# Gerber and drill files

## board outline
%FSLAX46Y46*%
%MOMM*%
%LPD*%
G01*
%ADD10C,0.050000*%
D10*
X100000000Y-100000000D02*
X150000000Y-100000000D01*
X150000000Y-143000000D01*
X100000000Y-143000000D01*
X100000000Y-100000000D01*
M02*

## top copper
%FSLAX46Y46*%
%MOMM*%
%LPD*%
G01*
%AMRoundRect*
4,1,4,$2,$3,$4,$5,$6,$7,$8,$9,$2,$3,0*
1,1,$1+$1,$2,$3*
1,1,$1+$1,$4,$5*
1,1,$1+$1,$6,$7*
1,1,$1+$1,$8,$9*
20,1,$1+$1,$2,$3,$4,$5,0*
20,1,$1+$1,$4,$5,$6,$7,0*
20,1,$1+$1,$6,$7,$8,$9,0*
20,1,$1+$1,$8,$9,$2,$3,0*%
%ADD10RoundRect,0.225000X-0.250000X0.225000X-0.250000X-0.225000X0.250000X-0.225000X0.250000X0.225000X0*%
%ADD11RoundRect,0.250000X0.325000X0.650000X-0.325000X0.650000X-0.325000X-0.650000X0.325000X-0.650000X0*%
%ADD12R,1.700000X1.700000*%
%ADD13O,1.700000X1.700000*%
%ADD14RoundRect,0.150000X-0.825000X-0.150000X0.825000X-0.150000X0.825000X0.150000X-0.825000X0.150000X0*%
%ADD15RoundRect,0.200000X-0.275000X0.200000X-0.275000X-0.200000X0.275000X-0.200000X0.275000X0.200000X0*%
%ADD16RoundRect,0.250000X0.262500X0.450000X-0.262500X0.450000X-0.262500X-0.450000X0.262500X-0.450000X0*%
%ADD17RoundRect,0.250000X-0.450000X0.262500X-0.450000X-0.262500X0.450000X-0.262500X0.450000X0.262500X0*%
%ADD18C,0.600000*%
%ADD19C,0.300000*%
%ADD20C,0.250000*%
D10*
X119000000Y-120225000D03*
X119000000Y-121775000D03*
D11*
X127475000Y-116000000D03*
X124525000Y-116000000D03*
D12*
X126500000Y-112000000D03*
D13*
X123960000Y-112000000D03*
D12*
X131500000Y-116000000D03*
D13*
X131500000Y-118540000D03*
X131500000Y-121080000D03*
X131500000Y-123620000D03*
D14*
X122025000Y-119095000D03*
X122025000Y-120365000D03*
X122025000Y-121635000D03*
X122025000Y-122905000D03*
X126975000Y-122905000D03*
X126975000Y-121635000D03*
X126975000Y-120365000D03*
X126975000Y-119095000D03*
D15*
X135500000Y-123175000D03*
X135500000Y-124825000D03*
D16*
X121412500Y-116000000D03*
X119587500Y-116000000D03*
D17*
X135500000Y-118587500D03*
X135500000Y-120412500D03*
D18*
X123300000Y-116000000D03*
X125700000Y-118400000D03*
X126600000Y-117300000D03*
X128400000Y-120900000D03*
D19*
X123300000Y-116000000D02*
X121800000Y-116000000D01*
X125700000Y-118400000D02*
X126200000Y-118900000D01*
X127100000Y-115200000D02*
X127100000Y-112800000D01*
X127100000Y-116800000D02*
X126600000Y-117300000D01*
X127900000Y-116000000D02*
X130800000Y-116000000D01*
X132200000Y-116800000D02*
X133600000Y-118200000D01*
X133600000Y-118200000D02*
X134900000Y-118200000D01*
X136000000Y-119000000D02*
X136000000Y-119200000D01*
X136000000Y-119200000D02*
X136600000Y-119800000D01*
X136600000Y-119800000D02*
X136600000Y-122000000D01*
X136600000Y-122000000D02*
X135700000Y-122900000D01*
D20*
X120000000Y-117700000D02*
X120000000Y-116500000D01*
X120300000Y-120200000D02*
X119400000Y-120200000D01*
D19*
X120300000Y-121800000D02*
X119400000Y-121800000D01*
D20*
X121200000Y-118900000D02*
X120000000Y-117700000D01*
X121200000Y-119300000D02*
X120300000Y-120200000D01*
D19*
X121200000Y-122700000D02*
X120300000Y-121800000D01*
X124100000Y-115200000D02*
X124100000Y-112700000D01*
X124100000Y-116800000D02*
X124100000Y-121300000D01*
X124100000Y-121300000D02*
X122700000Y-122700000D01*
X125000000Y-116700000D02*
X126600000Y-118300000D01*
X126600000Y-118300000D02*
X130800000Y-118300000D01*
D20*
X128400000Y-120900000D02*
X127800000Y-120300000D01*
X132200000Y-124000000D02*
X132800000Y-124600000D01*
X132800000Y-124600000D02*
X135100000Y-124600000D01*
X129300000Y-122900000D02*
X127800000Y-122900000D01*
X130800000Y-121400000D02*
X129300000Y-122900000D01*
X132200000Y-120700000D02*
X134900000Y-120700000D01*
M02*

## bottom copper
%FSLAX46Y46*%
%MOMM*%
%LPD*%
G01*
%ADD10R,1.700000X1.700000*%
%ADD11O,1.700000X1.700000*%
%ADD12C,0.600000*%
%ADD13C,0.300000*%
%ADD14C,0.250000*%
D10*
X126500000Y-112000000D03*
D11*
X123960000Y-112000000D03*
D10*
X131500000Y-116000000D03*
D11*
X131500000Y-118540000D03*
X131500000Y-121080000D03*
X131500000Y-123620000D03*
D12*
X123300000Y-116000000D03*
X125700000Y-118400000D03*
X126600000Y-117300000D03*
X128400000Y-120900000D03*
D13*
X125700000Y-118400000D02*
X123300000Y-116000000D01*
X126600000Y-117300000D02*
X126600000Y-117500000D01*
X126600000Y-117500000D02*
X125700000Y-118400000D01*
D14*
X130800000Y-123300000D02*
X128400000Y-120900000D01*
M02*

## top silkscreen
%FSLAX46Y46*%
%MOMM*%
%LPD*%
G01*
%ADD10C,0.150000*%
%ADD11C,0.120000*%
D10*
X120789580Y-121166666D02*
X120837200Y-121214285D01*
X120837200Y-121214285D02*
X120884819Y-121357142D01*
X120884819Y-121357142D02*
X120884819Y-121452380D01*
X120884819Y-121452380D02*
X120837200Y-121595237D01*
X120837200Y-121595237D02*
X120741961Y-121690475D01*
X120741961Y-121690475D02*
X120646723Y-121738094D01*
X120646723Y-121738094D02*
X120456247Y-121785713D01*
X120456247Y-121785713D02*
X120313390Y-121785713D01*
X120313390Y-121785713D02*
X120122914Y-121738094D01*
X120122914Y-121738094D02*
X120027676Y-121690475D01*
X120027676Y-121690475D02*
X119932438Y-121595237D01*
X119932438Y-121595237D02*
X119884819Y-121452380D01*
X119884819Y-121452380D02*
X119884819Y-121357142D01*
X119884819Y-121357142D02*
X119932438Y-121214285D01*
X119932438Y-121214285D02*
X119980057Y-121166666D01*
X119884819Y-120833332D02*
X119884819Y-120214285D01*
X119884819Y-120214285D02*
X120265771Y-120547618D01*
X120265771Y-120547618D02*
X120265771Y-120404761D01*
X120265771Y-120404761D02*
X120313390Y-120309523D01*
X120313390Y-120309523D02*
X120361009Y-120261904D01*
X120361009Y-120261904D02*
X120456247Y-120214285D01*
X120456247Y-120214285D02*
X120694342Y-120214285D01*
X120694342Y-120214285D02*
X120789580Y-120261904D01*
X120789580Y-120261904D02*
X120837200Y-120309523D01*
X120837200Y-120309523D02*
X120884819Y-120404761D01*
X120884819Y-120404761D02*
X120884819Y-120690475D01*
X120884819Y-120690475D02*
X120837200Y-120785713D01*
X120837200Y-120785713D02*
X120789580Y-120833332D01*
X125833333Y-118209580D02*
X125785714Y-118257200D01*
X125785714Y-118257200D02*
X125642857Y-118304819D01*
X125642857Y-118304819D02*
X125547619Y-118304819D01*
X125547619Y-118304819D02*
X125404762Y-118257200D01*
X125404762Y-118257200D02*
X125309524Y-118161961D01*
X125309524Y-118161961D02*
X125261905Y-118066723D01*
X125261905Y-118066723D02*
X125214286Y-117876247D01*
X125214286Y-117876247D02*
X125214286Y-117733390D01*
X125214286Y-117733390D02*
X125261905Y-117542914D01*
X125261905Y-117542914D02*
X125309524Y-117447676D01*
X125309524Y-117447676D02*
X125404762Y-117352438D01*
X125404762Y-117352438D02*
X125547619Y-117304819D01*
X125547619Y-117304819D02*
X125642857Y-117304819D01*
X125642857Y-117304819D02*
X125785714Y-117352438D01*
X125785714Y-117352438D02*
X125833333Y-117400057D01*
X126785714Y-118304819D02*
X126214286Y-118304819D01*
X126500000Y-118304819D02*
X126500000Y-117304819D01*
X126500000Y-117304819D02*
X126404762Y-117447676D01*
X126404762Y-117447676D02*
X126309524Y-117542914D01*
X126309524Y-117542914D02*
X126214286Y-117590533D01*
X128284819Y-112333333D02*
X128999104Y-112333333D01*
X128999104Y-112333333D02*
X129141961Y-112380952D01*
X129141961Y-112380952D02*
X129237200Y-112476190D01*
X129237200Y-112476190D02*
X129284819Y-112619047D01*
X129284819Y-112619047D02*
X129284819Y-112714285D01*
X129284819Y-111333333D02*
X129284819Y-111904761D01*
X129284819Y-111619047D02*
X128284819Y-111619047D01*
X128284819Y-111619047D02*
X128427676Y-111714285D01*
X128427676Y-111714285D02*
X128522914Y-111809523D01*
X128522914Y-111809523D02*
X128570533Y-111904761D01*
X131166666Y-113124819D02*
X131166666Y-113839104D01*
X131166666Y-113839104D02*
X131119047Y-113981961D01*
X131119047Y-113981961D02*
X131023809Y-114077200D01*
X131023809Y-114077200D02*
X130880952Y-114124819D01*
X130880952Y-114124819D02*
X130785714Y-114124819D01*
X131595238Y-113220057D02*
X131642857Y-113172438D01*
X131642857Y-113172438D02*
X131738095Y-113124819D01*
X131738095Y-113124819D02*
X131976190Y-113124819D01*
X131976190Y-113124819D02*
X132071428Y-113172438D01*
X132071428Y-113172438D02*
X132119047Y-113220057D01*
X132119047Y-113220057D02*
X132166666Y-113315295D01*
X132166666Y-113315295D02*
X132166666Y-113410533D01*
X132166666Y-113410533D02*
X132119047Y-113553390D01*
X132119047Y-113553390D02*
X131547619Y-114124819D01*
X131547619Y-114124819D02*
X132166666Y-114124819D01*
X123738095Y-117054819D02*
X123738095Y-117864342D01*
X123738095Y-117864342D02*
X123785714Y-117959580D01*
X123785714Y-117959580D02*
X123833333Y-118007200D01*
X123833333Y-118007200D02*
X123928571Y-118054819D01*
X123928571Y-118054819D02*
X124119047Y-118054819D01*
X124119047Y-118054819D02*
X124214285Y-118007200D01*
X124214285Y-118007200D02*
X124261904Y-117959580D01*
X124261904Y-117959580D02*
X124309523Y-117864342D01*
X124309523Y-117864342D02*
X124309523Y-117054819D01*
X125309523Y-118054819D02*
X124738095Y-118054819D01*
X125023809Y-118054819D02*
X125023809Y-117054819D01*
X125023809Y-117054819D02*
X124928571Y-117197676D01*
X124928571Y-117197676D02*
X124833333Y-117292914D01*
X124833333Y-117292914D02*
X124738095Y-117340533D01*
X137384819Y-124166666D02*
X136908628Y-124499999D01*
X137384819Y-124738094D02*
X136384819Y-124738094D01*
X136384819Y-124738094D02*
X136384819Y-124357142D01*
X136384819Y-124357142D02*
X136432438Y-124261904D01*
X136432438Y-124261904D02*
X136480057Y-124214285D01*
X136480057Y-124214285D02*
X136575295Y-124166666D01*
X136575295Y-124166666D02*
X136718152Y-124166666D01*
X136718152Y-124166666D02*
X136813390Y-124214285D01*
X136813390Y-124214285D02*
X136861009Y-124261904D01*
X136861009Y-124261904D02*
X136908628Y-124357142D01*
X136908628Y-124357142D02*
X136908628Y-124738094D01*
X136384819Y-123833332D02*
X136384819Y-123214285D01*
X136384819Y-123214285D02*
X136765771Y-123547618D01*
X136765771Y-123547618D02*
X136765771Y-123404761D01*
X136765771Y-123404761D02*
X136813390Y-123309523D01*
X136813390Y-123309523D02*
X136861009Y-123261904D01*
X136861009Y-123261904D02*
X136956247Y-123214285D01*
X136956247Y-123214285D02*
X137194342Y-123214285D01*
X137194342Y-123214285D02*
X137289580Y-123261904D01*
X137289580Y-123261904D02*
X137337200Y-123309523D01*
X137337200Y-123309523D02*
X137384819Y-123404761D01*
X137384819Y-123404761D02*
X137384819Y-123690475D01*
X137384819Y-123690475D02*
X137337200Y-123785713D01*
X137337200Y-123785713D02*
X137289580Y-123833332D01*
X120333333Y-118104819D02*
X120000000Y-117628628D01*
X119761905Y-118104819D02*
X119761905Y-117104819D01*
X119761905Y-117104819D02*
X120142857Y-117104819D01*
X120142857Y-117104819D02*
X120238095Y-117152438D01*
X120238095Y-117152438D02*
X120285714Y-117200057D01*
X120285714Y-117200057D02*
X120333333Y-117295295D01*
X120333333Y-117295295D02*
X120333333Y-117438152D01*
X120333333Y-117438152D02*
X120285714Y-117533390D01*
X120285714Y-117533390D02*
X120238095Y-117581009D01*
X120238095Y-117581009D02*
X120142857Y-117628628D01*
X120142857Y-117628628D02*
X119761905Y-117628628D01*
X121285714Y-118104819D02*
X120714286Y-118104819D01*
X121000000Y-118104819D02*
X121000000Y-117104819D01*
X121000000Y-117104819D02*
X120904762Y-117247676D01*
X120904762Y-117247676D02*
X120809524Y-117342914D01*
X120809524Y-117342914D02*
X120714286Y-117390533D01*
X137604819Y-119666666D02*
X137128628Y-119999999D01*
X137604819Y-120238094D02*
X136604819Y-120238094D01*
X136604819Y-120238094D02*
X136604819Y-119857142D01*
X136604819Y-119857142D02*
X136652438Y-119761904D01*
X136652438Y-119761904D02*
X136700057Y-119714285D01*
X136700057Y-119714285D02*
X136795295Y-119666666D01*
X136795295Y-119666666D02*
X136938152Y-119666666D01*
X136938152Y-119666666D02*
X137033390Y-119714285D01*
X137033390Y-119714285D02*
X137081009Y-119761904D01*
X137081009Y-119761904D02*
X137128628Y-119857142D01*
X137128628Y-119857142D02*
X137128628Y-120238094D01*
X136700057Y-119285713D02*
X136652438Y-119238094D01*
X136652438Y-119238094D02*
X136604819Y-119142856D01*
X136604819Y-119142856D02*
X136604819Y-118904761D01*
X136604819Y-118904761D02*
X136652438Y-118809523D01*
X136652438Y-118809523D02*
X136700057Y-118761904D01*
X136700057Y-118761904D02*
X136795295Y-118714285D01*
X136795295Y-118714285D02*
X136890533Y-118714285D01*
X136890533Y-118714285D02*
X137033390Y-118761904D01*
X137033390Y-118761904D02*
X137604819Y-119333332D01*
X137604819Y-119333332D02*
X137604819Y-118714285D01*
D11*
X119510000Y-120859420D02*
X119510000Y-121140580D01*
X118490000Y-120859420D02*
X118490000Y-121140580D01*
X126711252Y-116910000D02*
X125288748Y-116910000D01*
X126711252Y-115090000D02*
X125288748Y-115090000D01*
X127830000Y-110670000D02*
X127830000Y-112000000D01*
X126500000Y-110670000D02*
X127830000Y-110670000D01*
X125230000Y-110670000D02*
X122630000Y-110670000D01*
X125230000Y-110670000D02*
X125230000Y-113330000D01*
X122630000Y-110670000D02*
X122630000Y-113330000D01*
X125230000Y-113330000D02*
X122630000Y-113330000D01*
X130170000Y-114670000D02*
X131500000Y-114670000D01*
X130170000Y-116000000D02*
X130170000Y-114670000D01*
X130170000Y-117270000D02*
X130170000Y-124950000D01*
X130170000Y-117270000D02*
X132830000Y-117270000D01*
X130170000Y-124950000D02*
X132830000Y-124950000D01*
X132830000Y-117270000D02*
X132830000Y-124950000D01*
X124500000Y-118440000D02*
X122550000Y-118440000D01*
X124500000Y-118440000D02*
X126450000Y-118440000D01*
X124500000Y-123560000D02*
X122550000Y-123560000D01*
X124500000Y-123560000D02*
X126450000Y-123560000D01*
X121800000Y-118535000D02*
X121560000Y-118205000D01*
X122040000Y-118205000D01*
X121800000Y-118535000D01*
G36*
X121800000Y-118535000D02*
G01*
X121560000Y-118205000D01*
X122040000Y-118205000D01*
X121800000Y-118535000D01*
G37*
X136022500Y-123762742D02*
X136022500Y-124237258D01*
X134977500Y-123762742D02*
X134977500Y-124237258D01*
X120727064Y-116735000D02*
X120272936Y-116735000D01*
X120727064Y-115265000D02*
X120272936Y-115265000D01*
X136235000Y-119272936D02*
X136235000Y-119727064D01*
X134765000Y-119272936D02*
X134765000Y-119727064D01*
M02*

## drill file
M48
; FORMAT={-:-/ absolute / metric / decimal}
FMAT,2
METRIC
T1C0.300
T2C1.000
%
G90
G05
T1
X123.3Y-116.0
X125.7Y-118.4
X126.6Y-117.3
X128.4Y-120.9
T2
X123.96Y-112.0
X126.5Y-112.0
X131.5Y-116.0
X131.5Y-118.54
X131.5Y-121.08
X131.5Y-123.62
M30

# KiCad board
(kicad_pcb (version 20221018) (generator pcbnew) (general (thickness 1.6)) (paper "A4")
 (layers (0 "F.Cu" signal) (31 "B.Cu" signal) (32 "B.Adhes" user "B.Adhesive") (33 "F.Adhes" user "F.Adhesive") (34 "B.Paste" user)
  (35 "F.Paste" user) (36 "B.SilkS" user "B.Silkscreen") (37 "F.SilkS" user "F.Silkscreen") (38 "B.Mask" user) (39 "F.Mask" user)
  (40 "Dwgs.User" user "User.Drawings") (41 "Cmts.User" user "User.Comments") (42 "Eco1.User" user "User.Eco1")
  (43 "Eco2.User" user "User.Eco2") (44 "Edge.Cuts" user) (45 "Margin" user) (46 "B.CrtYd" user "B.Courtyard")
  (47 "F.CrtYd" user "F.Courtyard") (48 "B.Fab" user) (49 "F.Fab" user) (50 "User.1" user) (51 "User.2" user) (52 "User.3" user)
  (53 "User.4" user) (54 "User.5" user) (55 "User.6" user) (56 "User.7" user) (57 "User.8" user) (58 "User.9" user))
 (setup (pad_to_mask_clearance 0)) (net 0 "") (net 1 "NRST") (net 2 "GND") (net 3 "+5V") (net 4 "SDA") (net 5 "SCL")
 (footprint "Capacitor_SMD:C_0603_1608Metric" (layer "F.Cu") (at 119 121 -90)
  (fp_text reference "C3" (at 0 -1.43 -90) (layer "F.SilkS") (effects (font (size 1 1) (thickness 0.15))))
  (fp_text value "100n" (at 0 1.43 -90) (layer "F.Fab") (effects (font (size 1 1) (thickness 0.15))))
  (fp_line (start -0.14058 -0.51) (end 0.14058 -0.51) (stroke (width 0.12) (type solid)) (layer "F.SilkS"))
  (fp_line (start -0.14058 0.51) (end 0.14058 0.51) (stroke (width 0.12) (type solid)) (layer "F.SilkS"))
  (pad "1" smd roundrect (at -0.775 0 270) (size 0.9 0.95) (layers "F.Cu" "F.Paste" "F.Mask") (roundrect_rratio 0.25) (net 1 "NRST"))
  (pad "2" smd roundrect (at 0.775 0 270) (size 0.9 0.95) (layers "F.Cu" "F.Paste" "F.Mask") (roundrect_rratio 0.25) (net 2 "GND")))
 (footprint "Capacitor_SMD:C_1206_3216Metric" (layer "F.Cu") (at 126 116 180)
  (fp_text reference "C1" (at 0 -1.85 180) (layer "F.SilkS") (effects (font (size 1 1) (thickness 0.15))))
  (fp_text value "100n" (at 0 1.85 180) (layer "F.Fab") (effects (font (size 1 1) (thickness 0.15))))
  (fp_line (start -0.711252 -0.91) (end 0.711252 -0.91) (stroke (width 0.12) (type solid)) (layer "F.SilkS"))
  (fp_line (start -0.711252 0.91) (end 0.711252 0.91) (stroke (width 0.12) (type solid)) (layer "F.SilkS"))
  (pad "1" smd roundrect (at -1.475 0 180) (size 1.15 1.8) (layers "F.Cu" "F.Paste" "F.Mask") (roundrect_rratio 0.217391) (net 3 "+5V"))
  (pad "2" smd roundrect (at 1.475 0 180) (size 1.15 1.8) (layers "F.Cu" "F.Paste" "F.Mask") (roundrect_rratio 0.217391) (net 2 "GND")))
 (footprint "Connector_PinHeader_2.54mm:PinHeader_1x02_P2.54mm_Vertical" (layer "F.Cu") (at 126.5 112 -90)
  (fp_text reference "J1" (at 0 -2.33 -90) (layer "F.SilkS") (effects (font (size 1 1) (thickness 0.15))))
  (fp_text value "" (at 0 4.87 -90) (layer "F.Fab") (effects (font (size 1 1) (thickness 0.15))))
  (fp_line (start -1.33 -1.33) (end 0 -1.33) (stroke (width 0.12) (type solid)) (layer "F.SilkS"))
  (fp_line (start -1.33 0) (end -1.33 -1.33) (stroke (width 0.12) (type solid)) (layer "F.SilkS"))
  (fp_line (start -1.33 1.27) (end -1.33 3.87) (stroke (width 0.12) (type solid)) (layer "F.SilkS"))
  (fp_line (start -1.33 1.27) (end 1.33 1.27) (stroke (width 0.12) (type solid)) (layer "F.SilkS"))
  (fp_line (start -1.33 3.87) (end 1.33 3.87) (stroke (width 0.12) (type solid)) (layer "F.SilkS"))
  (fp_line (start 1.33 1.27) (end 1.33 3.87) (stroke (width 0.12) (type solid)) (layer "F.SilkS"))
  (pad "1" thru_hole rect (at 0 0 270) (size 1.7 1.7) (drill 1) (layers "*.Cu" "*.Mask") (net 3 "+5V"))
  (pad "2" thru_hole oval (at 0 2.54 270) (size 1.7 1.7) (drill 1) (layers "*.Cu" "*.Mask") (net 2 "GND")))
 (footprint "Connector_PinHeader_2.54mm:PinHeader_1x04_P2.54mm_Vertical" (layer "F.Cu") (at 131.5 116)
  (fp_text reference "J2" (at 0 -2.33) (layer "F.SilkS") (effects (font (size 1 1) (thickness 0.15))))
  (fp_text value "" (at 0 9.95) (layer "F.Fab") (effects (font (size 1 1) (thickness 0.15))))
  (fp_line (start -1.33 -1.33) (end 0 -1.33) (stroke (width 0.12) (type solid)) (layer "F.SilkS"))
  (fp_line (start -1.33 0) (end -1.33 -1.33) (stroke (width 0.12) (type solid)) (layer "F.SilkS"))
  (fp_line (start -1.33 1.27) (end -1.33 8.95) (stroke (width 0.12) (type solid)) (layer "F.SilkS"))
  (fp_line (start -1.33 1.27) (end 1.33 1.27) (stroke (width 0.12) (type solid)) (layer "F.SilkS"))
  (fp_line (start -1.33 8.95) (end 1.33 8.95) (stroke (width 0.12) (type solid)) (layer "F.SilkS"))
  (fp_line (start 1.33 1.27) (end 1.33 8.95) (stroke (width 0.12) (type solid)) (layer "F.SilkS"))
  (pad "1" thru_hole rect (at 0 0) (size 1.7 1.7) (drill 1) (layers "*.Cu" "*.Mask") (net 3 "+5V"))
  (pad "2" thru_hole oval (at 0 2.54) (size 1.7 1.7) (drill 1) (layers "*.Cu" "*.Mask") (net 2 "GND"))
  (pad "3" thru_hole oval (at 0 5.08) (size 1.7 1.7) (drill 1) (layers "*.Cu" "*.Mask") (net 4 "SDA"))
  (pad "4" thru_hole oval (at 0 7.62) (size 1.7 1.7) (drill 1) (layers "*.Cu" "*.Mask") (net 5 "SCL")))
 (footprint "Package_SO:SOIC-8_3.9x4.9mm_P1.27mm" (layer "F.Cu") (at 124.5 121)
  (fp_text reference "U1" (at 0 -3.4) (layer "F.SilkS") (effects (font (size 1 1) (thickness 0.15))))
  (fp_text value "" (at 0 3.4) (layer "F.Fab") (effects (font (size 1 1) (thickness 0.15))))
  (fp_line (start 0 -2.56) (end -1.95 -2.56) (stroke (width 0.12) (type solid)) (layer "F.SilkS"))
  (fp_line (start 0 -2.56) (end 1.95 -2.56) (stroke (width 0.12) (type solid)) (layer "F.SilkS"))
  (fp_line (start 0 2.56) (end -1.95 2.56) (stroke (width 0.12) (type solid)) (layer "F.SilkS"))
  (fp_line (start 0 2.56) (end 1.95 2.56) (stroke (width 0.12) (type solid)) (layer "F.SilkS"))
  (fp_poly
   (pts (xy -2.7 -2.465) (xy -2.94 -2.795) (xy -2.46 -2.795) (xy -2.7 -2.465)) (stroke (width 0.12) (type solid)) (fill solid)
   (layer "F.SilkS"))
  (pad "1" smd roundrect (at -2.475 -1.905) (size 1.95 0.6) (layers "F.Cu" "F.Paste" "F.Mask") (roundrect_rratio 0.25) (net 1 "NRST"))
  (pad "2" smd roundrect (at -2.475 -0.635) (size 1.95 0.6) (layers "F.Cu" "F.Paste" "F.Mask") (roundrect_rratio 0.25))
  (pad "3" smd roundrect (at -2.475 0.635) (size 1.95 0.6) (layers "F.Cu" "F.Paste" "F.Mask") (roundrect_rratio 0.25))
  (pad "4" smd roundrect (at -2.475 1.905) (size 1.95 0.6) (layers "F.Cu" "F.Paste" "F.Mask") (roundrect_rratio 0.25) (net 2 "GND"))
  (pad "5" smd roundrect (at 2.475 1.905) (size 1.95 0.6) (layers "F.Cu" "F.Paste" "F.Mask") (roundrect_rratio 0.25) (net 4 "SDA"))
  (pad "6" smd roundrect (at 2.475 0.635) (size 1.95 0.6) (layers "F.Cu" "F.Paste" "F.Mask") (roundrect_rratio 0.25))
  (pad "7" smd roundrect (at 2.475 -0.635) (size 1.95 0.6) (layers "F.Cu" "F.Paste" "F.Mask") (roundrect_rratio 0.25) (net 5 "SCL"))
  (pad "8" smd roundrect (at 2.475 -1.905) (size 1.95 0.6) (layers "F.Cu" "F.Paste" "F.Mask") (roundrect_rratio 0.25) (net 3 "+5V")))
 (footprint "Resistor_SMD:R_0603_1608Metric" (layer "F.Cu") (at 135.5 124 -90)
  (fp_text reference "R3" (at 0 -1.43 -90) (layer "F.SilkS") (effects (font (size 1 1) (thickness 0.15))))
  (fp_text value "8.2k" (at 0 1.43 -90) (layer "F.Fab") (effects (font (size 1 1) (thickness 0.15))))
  (fp_line (start -0.237258 -0.5225) (end 0.237258 -0.5225) (stroke (width 0.12) (type solid)) (layer "F.SilkS"))
  (fp_line (start -0.237258 0.5225) (end 0.237258 0.5225) (stroke (width 0.12) (type solid)) (layer "F.SilkS"))
  (pad "1" smd roundrect (at -0.825 0 270) (size 0.8 0.95) (layers "F.Cu" "F.Paste" "F.Mask") (roundrect_rratio 0.25) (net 3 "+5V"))
  (pad "2" smd roundrect (at 0.825 0 270) (size 0.8 0.95) (layers "F.Cu" "F.Paste" "F.Mask") (roundrect_rratio 0.25) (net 5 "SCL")))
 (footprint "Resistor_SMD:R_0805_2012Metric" (layer "F.Cu") (at 120.5 116 180)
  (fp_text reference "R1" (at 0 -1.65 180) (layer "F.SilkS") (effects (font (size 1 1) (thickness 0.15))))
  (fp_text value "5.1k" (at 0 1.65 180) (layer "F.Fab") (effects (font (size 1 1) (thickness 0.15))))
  (fp_line (start -0.227064 -0.735) (end 0.227064 -0.735) (stroke (width 0.12) (type solid)) (layer "F.SilkS"))
  (fp_line (start -0.227064 0.735) (end 0.227064 0.735) (stroke (width 0.12) (type solid)) (layer "F.SilkS"))
  (pad "1" smd roundrect (at -0.9125 0 180) (size 1.025 1.4) (layers "F.Cu" "F.Paste" "F.Mask") (roundrect_rratio 0.243902) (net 3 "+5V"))
  (pad "2" smd roundrect (at 0.9125 0 180) (size 1.025 1.4) (layers "F.Cu" "F.Paste" "F.Mask") (roundrect_rratio 0.243902) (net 1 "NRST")))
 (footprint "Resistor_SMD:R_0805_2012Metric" (layer "F.Cu") (at 135.5 119.5 -90)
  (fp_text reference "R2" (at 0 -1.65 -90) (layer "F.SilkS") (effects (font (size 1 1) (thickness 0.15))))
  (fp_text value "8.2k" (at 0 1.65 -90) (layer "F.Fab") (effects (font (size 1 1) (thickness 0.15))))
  (fp_line (start -0.227064 -0.735) (end 0.227064 -0.735) (stroke (width 0.12) (type solid)) (layer "F.SilkS"))
  (fp_line (start -0.227064 0.735) (end 0.227064 0.735) (stroke (width 0.12) (type solid)) (layer "F.SilkS"))
  (pad "1" smd roundrect (at -0.9125 0 270) (size 1.025 1.4) (layers "F.Cu" "F.Paste" "F.Mask") (roundrect_rratio 0.243902) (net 3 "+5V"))
  (pad "2" smd roundrect (at 0.9125 0 270) (size 1.025 1.4) (layers "F.Cu" "F.Paste" "F.Mask") (roundrect_rratio 0.243902) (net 4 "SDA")))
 (gr_rect (start 100 100) (end 150 143) (stroke (width 0.05) (type default)) (fill none) (layer "Edge.Cuts"))
 (segment (start 123.3 116) (end 121.8 116) (width 0.3) (layer "F.Cu") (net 3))
 (segment (start 125.7 118.4) (end 126.2 118.9) (width 0.3) (layer "F.Cu") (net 3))
 (segment (start 127.1 115.2) (end 127.1 112.8) (width 0.3) (layer "F.Cu") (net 3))
 (segment (start 127.1 116.8) (end 126.6 117.3) (width 0.3) (layer "F.Cu") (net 3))
 (segment (start 127.9 116) (end 130.8 116) (width 0.3) (layer "F.Cu") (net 3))
 (segment (start 132.2 116.8) (end 133.6 118.2) (width 0.3) (layer "F.Cu") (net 3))
 (segment (start 133.6 118.2) (end 134.9 118.2) (width 0.3) (layer "F.Cu") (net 3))
 (segment (start 136 119) (end 136 119.2) (width 0.3) (layer "F.Cu") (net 3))
 (segment (start 136 119.2) (end 136.6 119.8) (width 0.3) (layer "F.Cu") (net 3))
 (segment (start 136.6 119.8) (end 136.6 122) (width 0.3) (layer "F.Cu") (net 3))
 (segment (start 136.6 122) (end 135.7 122.9) (width 0.3) (layer "F.Cu") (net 3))
 (via (at 123.3 116) (size 0.6) (drill 0.3) (layers "F.Cu" "B.Cu") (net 3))
 (via (at 125.7 118.4) (size 0.6) (drill 0.3) (layers "F.Cu" "B.Cu") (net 3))
 (via (at 126.6 117.3) (size 0.6) (drill 0.3) (layers "F.Cu" "B.Cu") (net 3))
 (segment (start 120 117.7) (end 120 116.5) (width 0.25) (layer "F.Cu") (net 1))
 (segment (start 120.3 120.2) (end 119.4 120.2) (width 0.25) (layer "F.Cu") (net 1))
 (segment (start 120.3 121.8) (end 119.4 121.8) (width 0.3) (layer "F.Cu") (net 2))
 (segment (start 121.2 118.9) (end 120 117.7) (width 0.25) (layer "F.Cu") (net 1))
 (segment (start 121.2 119.3) (end 120.3 120.2) (width 0.25) (layer "F.Cu") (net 1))
 (segment (start 121.2 122.7) (end 120.3 121.8) (width 0.3) (layer "F.Cu") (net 2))
 (segment (start 124.1 115.2) (end 124.1 112.7) (width 0.3) (layer "F.Cu") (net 2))
 (segment (start 124.1 116.8) (end 124.1 121.3) (width 0.3) (layer "F.Cu") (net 2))
 (segment (start 124.1 121.3) (end 122.7 122.7) (width 0.3) (layer "F.Cu") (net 2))
 (segment (start 125 116.7) (end 126.6 118.3) (width 0.3) (layer "F.Cu") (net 2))
 (segment (start 125.7 118.4) (end 123.3 116) (width 0.3) (layer "B.Cu") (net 3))
 (segment (start 126.6 117.3) (end 126.6 117.5) (width 0.3) (layer "B.Cu") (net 3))
 (segment (start 126.6 117.5) (end 125.7 118.4) (width 0.3) (layer "B.Cu") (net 3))
 (segment (start 126.6 118.3) (end 130.8 118.3) (width 0.3) (layer "F.Cu") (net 2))
 (segment (start 128.4 120.9) (end 127.8 120.3) (width 0.25) (layer "F.Cu") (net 5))
 (segment (start 132.2 124) (end 132.8 124.6) (width 0.25) (layer "F.Cu") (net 5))
 (segment (start 132.8 124.6) (end 135.1 124.6) (width 0.25) (layer "F.Cu") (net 5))
 (via (at 128.4 120.9) (size 0.6) (drill 0.3) (layers "F.Cu" "B.Cu") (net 5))
 (segment (start 129.3 122.9) (end 127.8 122.9) (width 0.25) (layer "F.Cu") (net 4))
 (segment (start 130.8 121.4) (end 129.3 122.9) (width 0.25) (layer "F.Cu") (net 4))
 (segment (start 130.8 123.3) (end 128.4 120.9) (width 0.25) (layer "B.Cu") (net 5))
 (segment (start 132.2 120.7) (end 134.9 120.7) (width 0.25) (layer "F.Cu") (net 4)))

